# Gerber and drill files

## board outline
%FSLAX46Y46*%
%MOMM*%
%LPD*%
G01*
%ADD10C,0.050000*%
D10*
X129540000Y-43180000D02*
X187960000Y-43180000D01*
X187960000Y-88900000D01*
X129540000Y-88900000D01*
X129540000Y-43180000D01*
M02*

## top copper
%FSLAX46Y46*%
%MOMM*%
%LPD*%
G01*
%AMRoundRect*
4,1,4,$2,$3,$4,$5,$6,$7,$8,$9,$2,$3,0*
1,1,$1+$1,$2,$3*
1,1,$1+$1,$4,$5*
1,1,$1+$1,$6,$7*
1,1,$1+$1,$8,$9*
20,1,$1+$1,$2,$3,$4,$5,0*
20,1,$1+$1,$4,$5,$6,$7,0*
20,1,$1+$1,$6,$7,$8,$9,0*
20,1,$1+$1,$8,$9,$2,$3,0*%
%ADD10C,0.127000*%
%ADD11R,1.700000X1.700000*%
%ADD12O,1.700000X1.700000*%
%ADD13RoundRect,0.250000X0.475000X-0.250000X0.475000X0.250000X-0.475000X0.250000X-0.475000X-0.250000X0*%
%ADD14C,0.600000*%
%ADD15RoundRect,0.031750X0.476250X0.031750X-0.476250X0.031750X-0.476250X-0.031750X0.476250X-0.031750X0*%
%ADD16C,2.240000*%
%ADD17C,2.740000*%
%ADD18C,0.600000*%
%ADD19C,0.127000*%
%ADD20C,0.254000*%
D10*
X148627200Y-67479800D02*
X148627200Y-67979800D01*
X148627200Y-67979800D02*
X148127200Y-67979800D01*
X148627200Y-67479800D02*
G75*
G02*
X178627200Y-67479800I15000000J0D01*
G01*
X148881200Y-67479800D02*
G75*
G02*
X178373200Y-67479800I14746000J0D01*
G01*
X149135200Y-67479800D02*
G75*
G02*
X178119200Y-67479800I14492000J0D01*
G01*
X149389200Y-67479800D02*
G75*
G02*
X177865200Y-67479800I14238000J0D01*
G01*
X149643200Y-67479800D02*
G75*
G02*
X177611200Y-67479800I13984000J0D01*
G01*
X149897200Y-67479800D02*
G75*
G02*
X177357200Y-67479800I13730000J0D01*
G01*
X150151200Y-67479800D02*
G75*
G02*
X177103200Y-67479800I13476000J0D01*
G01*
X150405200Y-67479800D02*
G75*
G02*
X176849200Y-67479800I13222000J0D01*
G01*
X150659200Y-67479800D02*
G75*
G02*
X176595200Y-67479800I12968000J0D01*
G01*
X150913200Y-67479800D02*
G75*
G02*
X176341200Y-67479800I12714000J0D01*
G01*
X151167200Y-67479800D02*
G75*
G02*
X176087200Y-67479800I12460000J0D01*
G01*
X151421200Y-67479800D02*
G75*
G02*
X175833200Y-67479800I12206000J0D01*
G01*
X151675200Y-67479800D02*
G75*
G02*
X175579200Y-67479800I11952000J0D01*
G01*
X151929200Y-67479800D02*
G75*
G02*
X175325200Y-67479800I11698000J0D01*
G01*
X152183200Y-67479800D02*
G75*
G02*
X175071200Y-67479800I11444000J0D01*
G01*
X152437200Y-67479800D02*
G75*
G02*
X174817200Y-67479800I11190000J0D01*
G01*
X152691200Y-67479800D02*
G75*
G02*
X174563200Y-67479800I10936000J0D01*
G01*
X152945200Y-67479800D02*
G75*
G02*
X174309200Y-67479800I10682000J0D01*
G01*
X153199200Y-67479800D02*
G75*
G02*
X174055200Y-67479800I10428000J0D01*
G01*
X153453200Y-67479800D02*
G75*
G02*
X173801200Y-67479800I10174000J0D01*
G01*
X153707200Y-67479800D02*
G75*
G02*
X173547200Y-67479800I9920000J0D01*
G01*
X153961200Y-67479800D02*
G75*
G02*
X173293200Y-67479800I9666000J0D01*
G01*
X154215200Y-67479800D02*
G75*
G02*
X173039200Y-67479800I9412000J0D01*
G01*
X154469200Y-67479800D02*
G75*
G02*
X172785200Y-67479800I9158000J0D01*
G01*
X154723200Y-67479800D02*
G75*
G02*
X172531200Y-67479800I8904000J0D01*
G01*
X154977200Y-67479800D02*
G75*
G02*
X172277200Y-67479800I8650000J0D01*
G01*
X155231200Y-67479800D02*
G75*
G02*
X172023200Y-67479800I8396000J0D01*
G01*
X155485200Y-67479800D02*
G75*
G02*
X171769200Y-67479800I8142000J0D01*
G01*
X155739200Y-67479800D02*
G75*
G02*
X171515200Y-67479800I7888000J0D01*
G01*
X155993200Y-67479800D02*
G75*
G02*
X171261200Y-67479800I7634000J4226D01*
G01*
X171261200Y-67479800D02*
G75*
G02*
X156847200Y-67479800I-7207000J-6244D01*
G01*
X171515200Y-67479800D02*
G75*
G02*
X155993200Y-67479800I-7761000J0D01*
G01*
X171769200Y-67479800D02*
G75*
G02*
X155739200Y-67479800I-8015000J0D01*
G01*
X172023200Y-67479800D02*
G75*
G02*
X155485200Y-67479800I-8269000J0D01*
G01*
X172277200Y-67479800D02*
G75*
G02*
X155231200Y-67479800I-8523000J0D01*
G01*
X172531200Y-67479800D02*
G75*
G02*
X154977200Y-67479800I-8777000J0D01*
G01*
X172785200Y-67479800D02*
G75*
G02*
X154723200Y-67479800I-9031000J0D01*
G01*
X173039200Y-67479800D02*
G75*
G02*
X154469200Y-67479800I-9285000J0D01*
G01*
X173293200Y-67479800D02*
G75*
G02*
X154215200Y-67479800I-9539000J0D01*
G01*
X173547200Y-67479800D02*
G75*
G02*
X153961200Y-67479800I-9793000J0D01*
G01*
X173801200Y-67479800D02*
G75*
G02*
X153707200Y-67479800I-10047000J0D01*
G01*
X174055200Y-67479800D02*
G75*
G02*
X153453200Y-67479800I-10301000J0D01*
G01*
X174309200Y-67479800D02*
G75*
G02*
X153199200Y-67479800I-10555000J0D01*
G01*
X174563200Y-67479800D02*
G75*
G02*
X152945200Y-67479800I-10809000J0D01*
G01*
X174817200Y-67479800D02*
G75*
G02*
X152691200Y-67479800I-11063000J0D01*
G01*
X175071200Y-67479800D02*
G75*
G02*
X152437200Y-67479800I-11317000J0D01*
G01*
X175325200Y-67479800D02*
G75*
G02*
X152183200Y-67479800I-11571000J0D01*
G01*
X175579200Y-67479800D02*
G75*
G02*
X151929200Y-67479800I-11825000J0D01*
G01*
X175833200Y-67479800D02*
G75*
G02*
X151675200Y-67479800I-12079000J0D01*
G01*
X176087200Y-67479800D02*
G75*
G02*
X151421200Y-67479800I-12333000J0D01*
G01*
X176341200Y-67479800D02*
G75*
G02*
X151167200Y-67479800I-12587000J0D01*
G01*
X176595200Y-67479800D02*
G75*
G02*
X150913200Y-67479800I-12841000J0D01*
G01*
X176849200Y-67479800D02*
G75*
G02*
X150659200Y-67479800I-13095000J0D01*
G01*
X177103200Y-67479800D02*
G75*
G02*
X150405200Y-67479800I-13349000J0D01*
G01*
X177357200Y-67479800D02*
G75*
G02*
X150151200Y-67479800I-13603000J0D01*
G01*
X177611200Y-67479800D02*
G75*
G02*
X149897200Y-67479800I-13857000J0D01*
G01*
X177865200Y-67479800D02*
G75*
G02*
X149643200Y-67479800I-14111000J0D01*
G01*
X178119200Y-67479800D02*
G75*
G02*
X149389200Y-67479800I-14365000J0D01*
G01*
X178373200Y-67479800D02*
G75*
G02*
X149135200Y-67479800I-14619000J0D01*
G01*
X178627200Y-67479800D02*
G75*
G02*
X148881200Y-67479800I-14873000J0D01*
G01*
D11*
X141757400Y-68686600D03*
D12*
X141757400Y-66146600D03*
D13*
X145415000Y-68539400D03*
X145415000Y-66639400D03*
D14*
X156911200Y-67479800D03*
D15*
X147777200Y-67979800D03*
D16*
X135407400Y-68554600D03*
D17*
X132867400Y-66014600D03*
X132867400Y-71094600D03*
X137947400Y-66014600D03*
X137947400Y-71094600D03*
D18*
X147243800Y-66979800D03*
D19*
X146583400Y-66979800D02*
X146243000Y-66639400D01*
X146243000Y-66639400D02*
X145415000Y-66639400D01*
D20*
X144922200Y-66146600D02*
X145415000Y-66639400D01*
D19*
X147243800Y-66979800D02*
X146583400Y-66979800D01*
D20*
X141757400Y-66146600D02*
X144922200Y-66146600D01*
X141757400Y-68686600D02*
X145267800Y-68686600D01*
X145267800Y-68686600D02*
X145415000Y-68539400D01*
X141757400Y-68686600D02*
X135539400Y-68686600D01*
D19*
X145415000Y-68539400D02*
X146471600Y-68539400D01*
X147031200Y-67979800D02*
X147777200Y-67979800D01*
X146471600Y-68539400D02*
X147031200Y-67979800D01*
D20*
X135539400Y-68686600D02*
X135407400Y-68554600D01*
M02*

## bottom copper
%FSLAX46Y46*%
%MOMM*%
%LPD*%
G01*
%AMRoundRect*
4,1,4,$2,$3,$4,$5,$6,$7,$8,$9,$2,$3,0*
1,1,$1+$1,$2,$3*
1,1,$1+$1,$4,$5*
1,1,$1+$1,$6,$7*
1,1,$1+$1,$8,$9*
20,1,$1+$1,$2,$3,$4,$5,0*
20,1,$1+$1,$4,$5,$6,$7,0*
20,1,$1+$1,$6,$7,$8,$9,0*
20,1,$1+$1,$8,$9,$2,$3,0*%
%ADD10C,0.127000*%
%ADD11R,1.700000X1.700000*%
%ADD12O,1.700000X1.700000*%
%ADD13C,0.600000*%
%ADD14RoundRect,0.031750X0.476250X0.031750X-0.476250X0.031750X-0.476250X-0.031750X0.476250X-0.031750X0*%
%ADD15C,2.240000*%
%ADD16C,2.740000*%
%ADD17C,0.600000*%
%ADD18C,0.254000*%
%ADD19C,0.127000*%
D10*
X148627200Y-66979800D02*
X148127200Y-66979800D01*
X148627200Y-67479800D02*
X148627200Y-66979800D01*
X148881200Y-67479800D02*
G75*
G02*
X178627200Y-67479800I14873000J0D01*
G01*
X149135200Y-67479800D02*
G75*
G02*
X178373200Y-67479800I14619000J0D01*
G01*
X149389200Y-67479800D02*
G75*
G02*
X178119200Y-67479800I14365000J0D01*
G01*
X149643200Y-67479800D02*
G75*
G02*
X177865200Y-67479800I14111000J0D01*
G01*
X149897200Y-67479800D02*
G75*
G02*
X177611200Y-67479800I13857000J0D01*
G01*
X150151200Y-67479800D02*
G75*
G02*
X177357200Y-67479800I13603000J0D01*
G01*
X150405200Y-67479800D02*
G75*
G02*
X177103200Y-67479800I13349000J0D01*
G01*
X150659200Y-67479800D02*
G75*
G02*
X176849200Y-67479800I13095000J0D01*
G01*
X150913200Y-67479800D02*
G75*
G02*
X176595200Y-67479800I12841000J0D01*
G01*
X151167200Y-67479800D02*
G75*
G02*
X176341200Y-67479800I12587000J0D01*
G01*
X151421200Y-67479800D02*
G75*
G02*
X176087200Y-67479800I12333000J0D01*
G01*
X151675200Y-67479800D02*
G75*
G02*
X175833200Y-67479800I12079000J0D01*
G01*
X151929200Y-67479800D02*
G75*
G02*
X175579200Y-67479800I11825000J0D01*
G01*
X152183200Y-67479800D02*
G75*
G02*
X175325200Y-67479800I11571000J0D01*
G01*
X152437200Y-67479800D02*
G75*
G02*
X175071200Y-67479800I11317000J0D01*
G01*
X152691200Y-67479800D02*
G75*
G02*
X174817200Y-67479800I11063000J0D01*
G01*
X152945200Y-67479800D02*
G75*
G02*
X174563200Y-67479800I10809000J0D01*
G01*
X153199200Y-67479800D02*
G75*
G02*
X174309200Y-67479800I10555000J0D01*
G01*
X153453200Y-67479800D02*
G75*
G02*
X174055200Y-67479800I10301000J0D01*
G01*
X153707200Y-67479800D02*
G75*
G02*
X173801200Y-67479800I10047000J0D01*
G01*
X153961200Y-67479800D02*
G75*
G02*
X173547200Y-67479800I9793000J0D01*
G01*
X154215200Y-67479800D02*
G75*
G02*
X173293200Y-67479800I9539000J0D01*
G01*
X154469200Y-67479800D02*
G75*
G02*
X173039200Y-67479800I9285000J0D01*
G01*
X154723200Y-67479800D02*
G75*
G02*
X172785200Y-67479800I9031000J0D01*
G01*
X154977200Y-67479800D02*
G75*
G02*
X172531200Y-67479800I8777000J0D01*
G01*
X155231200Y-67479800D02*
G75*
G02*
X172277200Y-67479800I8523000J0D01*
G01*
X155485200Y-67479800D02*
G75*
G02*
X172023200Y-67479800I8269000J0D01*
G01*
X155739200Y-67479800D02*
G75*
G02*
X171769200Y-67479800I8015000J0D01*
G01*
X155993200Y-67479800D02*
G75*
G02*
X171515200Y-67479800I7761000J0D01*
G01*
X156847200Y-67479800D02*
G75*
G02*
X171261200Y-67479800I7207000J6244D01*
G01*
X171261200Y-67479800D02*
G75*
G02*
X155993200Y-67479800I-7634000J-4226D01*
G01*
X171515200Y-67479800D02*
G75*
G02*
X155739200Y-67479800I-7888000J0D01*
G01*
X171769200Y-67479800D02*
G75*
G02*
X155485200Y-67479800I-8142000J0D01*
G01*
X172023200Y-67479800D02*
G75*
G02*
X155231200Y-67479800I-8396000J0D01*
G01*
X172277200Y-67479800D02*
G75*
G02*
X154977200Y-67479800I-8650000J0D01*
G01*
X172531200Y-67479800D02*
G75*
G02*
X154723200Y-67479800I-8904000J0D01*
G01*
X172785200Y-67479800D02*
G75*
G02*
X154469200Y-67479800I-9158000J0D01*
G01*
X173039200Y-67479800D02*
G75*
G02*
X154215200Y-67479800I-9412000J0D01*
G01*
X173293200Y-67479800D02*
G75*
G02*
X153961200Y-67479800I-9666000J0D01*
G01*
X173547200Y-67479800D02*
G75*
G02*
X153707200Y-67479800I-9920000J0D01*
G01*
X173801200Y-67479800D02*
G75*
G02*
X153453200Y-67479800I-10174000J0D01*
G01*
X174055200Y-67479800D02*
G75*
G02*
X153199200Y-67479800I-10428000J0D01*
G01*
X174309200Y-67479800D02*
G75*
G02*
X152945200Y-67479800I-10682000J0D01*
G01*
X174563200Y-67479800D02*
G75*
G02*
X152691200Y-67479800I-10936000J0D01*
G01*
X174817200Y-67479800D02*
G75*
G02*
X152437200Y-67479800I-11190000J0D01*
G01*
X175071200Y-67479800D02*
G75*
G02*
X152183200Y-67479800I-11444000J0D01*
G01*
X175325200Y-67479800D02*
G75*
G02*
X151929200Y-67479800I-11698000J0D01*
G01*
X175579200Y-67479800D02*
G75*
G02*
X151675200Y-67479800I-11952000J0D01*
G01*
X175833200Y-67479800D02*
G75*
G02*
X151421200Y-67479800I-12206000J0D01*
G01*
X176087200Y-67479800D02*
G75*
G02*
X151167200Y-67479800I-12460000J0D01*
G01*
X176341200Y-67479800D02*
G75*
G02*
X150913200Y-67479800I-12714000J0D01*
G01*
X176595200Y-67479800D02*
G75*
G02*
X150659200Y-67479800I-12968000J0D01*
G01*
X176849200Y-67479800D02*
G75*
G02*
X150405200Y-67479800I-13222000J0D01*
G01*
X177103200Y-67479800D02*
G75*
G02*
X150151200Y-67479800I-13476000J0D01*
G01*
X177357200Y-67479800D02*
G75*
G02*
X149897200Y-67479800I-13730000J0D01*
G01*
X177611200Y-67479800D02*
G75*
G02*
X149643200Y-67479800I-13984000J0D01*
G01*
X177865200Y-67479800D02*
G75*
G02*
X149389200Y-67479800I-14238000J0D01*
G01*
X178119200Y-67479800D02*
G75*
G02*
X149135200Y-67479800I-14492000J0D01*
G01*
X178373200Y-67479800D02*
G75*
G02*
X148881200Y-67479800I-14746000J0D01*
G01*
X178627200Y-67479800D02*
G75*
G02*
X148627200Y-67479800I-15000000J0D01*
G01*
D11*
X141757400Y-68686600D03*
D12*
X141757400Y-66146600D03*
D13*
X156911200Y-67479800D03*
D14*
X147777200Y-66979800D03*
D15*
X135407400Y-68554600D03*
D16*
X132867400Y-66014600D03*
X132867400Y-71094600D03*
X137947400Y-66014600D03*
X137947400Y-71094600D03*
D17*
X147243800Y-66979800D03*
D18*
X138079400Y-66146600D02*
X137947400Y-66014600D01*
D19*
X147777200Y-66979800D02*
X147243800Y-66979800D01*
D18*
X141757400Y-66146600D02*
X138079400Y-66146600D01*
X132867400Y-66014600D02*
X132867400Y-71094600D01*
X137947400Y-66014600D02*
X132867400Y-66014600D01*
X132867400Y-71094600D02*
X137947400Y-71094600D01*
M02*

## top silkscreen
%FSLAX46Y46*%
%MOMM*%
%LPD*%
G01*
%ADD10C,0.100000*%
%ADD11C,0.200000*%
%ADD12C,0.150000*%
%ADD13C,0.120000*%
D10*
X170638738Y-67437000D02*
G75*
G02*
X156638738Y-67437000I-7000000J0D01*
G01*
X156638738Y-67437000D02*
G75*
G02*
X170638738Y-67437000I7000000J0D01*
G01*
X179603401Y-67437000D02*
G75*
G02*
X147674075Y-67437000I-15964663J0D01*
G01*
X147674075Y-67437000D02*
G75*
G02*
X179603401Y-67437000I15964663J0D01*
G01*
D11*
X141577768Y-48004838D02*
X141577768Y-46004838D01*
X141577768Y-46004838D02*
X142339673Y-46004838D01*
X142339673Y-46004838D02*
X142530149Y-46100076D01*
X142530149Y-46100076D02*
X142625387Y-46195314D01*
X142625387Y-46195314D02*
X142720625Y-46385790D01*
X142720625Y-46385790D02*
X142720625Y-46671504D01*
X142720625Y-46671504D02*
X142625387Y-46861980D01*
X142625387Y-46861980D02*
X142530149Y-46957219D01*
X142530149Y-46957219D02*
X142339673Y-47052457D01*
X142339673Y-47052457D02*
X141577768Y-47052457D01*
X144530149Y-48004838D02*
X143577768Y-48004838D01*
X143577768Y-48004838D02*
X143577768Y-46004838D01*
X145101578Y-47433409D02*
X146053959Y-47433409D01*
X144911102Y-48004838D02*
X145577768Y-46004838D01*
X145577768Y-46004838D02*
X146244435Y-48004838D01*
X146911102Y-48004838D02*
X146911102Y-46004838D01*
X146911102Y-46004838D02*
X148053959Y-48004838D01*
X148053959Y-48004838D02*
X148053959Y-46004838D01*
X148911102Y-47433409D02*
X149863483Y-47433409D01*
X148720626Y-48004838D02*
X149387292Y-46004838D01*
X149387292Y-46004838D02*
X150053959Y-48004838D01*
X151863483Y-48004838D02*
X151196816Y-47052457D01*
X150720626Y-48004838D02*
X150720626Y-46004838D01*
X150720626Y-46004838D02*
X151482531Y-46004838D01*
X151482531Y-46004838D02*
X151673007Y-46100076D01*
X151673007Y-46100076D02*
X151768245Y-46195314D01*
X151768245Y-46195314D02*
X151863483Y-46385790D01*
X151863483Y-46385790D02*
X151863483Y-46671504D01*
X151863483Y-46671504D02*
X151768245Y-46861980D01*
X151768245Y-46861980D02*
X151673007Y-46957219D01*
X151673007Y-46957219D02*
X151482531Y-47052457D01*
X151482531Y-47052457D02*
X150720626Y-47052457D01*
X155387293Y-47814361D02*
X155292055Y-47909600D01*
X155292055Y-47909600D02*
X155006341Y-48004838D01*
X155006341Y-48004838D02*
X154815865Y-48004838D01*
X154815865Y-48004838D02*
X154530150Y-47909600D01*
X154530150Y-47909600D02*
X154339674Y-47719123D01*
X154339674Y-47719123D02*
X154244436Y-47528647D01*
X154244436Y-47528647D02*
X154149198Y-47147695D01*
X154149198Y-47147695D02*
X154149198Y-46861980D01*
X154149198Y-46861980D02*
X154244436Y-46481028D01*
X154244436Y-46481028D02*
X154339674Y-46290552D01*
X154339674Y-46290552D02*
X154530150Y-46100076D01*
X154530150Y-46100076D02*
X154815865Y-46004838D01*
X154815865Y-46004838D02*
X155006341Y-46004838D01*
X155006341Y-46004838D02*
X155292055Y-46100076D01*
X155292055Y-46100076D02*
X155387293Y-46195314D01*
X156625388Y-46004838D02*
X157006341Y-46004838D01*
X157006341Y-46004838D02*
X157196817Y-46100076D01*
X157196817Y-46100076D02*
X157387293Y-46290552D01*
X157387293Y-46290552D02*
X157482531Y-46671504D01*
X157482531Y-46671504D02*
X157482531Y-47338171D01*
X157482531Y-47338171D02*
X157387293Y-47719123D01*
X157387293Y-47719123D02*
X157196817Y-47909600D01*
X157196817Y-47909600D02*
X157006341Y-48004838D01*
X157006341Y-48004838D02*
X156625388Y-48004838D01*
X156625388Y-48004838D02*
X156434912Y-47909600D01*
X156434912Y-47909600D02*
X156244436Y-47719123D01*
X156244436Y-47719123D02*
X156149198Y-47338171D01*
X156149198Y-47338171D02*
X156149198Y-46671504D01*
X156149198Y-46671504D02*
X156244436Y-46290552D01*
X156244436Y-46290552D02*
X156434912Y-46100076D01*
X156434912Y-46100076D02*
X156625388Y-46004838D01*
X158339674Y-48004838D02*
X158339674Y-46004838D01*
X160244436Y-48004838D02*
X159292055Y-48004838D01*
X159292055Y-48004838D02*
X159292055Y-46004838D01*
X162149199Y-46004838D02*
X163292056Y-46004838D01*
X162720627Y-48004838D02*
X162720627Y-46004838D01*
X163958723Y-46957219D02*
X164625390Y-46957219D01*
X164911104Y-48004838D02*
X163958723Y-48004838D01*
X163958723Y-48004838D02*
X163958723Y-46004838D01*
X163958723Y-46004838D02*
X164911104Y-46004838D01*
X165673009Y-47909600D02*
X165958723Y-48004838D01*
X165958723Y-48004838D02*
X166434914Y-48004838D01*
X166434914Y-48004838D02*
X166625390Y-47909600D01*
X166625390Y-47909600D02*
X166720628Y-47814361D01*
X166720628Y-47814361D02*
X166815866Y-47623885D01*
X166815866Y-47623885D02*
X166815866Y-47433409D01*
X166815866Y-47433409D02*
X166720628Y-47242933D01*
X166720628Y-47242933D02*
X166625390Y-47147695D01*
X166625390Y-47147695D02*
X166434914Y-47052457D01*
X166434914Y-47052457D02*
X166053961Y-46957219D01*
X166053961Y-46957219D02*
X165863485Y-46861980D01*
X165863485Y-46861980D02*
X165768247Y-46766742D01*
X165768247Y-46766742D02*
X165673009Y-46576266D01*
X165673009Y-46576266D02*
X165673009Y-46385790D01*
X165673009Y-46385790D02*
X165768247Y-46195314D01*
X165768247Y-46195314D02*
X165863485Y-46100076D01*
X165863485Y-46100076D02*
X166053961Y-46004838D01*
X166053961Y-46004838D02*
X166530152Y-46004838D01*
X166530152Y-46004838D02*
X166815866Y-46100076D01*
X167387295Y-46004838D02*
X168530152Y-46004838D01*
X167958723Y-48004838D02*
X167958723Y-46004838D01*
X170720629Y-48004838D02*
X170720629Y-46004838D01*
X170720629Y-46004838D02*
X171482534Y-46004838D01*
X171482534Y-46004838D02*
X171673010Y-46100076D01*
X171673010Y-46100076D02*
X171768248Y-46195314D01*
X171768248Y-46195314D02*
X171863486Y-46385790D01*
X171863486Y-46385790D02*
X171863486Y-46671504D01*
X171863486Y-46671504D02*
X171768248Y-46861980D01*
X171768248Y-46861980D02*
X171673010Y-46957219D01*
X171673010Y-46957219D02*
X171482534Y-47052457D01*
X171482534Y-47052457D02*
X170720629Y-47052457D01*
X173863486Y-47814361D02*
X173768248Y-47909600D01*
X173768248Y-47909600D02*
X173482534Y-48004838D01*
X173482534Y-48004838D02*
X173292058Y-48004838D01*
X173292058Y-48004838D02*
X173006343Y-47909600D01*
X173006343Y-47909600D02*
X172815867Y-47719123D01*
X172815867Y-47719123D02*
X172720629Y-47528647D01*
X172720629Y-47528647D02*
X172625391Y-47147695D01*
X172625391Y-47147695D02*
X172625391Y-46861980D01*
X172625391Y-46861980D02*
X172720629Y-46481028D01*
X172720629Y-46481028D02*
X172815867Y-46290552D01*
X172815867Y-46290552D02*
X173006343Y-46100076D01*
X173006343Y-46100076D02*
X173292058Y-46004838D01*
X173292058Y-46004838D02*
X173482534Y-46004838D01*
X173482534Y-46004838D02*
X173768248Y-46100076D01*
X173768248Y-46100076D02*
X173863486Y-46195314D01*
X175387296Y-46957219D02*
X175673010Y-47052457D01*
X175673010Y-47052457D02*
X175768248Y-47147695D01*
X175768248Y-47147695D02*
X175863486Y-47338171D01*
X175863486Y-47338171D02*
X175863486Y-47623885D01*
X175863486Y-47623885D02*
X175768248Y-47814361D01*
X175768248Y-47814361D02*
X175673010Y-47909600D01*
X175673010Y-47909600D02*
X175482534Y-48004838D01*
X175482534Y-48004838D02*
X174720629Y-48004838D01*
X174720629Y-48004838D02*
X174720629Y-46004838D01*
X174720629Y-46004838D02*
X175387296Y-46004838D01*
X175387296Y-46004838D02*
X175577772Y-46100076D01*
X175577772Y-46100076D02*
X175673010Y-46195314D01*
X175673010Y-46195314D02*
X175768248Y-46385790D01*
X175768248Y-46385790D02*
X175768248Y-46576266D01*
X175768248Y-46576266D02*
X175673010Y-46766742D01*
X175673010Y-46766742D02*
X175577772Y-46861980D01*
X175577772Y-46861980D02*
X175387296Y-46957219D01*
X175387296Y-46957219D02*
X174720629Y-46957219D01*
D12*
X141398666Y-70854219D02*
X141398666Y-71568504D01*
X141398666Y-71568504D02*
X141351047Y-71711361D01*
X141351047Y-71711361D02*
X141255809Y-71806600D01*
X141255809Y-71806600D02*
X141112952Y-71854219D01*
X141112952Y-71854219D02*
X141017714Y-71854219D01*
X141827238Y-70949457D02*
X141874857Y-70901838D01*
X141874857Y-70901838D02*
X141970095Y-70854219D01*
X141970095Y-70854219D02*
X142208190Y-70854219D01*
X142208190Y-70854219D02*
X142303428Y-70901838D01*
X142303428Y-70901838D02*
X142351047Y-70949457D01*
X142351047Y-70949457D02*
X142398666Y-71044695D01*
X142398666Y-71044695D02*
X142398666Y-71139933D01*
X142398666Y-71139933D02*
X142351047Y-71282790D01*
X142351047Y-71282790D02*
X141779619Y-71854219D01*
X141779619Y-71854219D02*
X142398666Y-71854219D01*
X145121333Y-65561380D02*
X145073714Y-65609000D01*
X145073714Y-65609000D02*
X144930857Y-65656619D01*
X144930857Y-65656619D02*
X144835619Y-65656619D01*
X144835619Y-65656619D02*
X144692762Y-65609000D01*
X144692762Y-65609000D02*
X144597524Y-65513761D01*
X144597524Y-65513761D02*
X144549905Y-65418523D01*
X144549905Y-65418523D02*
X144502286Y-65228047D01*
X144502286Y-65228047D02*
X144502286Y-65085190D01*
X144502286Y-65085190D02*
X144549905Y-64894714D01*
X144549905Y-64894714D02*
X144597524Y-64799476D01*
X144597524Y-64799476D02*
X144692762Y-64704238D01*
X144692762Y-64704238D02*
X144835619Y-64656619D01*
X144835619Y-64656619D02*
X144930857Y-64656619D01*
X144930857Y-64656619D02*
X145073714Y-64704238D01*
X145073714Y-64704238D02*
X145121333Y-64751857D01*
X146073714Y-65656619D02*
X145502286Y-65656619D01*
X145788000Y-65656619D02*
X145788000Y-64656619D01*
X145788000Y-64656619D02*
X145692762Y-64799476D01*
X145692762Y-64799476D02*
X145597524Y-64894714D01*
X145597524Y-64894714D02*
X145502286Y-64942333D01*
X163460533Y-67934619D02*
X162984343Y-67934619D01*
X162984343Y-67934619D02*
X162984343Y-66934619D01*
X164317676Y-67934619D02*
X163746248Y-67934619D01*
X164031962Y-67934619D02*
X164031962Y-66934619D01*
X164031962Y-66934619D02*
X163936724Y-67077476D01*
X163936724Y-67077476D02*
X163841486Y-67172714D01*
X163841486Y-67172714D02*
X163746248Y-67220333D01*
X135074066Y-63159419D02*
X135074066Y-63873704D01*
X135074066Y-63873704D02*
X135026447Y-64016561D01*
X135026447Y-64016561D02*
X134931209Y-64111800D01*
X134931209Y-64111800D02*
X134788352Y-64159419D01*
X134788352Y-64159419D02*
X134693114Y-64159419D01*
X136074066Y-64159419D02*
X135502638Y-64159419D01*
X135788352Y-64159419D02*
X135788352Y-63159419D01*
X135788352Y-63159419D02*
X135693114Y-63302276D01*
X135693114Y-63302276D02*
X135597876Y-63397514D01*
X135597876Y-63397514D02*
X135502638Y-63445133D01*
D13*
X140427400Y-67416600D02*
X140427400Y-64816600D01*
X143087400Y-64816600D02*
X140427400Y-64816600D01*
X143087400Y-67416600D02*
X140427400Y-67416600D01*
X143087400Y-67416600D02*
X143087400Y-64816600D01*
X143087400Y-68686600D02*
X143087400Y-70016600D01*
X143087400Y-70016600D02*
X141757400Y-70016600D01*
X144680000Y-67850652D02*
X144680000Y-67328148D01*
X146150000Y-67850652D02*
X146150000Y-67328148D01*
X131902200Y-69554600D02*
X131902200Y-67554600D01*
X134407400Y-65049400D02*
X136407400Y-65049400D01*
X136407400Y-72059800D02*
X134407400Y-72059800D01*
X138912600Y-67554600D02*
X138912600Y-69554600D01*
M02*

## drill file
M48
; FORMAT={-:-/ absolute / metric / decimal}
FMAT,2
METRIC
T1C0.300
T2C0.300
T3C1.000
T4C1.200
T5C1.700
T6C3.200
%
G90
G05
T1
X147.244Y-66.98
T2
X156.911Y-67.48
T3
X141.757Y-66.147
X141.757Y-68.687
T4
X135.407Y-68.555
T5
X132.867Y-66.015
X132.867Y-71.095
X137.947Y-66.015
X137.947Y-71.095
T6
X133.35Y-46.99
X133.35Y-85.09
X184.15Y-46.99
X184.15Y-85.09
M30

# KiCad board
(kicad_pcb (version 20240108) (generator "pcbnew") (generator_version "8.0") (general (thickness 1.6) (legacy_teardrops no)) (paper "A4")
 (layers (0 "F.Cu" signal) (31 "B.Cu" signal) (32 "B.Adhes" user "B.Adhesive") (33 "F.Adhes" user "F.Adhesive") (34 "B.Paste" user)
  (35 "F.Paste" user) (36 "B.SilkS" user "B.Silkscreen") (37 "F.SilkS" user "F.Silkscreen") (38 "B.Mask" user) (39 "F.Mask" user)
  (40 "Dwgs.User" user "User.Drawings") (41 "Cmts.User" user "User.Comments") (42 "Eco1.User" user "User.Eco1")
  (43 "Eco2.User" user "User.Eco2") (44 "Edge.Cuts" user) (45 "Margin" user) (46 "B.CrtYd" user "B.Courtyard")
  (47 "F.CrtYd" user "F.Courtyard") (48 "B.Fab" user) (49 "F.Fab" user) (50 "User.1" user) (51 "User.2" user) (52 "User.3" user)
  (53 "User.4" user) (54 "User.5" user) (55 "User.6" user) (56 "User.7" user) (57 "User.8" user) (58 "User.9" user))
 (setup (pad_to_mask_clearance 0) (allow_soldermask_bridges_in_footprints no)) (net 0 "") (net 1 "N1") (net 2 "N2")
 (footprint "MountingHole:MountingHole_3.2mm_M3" (layer "F.Cu") (at 184.15 85.09)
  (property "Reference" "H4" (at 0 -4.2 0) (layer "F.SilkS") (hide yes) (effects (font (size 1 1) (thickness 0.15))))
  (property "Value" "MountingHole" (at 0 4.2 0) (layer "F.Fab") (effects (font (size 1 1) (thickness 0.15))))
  (pad "" np_thru_hole circle (at 0 0) (size 3.2 3.2) (drill 3.2) (layers "*.Cu" "*.Mask")))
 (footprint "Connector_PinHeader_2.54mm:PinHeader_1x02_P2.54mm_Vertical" (layer "F.Cu") (at 141.7574 68.6866 180)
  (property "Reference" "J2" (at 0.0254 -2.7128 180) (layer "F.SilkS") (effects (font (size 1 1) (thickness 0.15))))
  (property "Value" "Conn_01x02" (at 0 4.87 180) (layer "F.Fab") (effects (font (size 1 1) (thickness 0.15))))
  (fp_line (start 1.33 1.27) (end 1.33 3.87) (stroke (width 0.12) (type solid)) (layer "F.SilkS"))
  (fp_line (start -1.33 3.87) (end 1.33 3.87) (stroke (width 0.12) (type solid)) (layer "F.SilkS"))
  (fp_line (start -1.33 1.27) (end 1.33 1.27) (stroke (width 0.12) (type solid)) (layer "F.SilkS"))
  (fp_line (start -1.33 1.27) (end -1.33 3.87) (stroke (width 0.12) (type solid)) (layer "F.SilkS"))
  (fp_line (start -1.33 0) (end -1.33 -1.33) (stroke (width 0.12) (type solid)) (layer "F.SilkS"))
  (fp_line (start -1.33 -1.33) (end 0 -1.33) (stroke (width 0.12) (type solid)) (layer "F.SilkS"))
  (pad "1" thru_hole rect (at 0 0 180) (size 1.7 1.7) (drill 1) (layers "*.Cu" "*.Mask") (remove_unused_layers no) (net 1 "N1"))
  (pad "2" thru_hole oval (at 0 2.54 180) (size 1.7 1.7) (drill 1) (layers "*.Cu" "*.Mask") (remove_unused_layers no) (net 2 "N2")))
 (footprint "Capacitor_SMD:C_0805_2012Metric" (layer "F.Cu") (at 145.415 67.5894 90)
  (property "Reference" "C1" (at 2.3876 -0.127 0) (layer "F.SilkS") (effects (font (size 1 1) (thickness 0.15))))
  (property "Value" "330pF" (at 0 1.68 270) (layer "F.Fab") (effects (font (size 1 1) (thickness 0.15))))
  (fp_line (start -0.261252 -0.735) (end 0.261252 -0.735) (stroke (width 0.12) (type solid)) (layer "F.SilkS"))
  (fp_line (start -0.261252 0.735) (end 0.261252 0.735) (stroke (width 0.12) (type solid)) (layer "F.SilkS"))
  (pad "1" smd roundrect (at -0.95 0 90) (size 1 1.45) (layers "F.Cu" "F.Paste" "F.Mask") (roundrect_rratio 0.25) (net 1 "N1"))
  (pad "2" smd roundrect (at 0.95 0 90) (size 1 1.45) (layers "F.Cu" "F.Paste" "F.Mask") (roundrect_rratio 0.25) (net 2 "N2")))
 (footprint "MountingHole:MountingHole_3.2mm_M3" (layer "F.Cu") (at 133.35 46.99)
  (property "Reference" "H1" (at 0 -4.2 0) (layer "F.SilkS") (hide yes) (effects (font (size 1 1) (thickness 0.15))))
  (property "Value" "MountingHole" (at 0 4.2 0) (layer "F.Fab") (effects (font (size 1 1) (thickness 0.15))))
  (pad "" np_thru_hole circle (at 0 0) (size 3.2 3.2) (drill 3.2) (layers "*.Cu" "*.Mask")))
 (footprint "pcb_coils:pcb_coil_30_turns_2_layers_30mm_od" (layer "F.Cu") (at 163.7542 67.4798 180)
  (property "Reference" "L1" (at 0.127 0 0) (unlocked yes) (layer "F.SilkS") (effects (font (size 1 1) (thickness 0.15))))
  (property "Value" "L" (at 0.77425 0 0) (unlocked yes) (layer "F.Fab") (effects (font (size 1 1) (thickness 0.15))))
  (fp_line (start 15.127 0) (end 15.127 -0.5) (stroke (width 0.127) (type solid)) (layer "F.Cu"))
  (fp_line (start 15.127 -0.5) (end 15.627 -0.5) (stroke (width 0.127) (type solid)) (layer "F.Cu"))
  (fp_arc (start 15.127 0) (mid 0.127 15) (end -14.873 0) (stroke (width 0.127) (type solid)) (layer "F.Cu"))
  (fp_arc (start 14.873 0) (mid 0.127 14.746) (end -14.619 0) (stroke (width 0.127) (type solid)) (layer "F.Cu"))
  (fp_arc (start 14.619 0) (mid 0.127 14.492) (end -14.365 0) (stroke (width 0.127) (type solid)) (layer "F.Cu"))
  (fp_arc (start 14.365 0) (mid 0.127 14.238) (end -14.111 0) (stroke (width 0.127) (type solid)) (layer "F.Cu"))
  (fp_arc (start 14.111 0) (mid 0.127 13.984) (end -13.857 0) (stroke (width 0.127) (type solid)) (layer "F.Cu"))
  (fp_arc (start 13.857 0) (mid 0.127 13.73) (end -13.603 0) (stroke (width 0.127) (type solid)) (layer "F.Cu"))
  (fp_arc (start 13.603 0) (mid 0.127 13.476) (end -13.349 0) (stroke (width 0.127) (type solid)) (layer "F.Cu"))
  (fp_arc (start 13.349 0) (mid 0.127 13.222) (end -13.095 0) (stroke (width 0.127) (type solid)) (layer "F.Cu"))
  (fp_arc (start 13.095 0) (mid 0.127 12.968) (end -12.841 0) (stroke (width 0.127) (type solid)) (layer "F.Cu"))
  (fp_arc (start 12.841 0) (mid 0.127 12.714) (end -12.587 0) (stroke (width 0.127) (type solid)) (layer "F.Cu"))
  (fp_arc (start 12.587 0) (mid 0.127 12.46) (end -12.333 0) (stroke (width 0.127) (type solid)) (layer "F.Cu"))
  (fp_arc (start 12.333 0) (mid 0.127 12.206) (end -12.079 0) (stroke (width 0.127) (type solid)) (layer "F.Cu"))
  (fp_arc (start 12.079 0) (mid 0.127 11.952) (end -11.825 0) (stroke (width 0.127) (type solid)) (layer "F.Cu"))
  (fp_arc (start 11.825 0) (mid 0.127 11.698) (end -11.571 0) (stroke (width 0.127) (type solid)) (layer "F.Cu"))
  (fp_arc (start 11.571 0) (mid 0.127 11.444) (end -11.317 0) (stroke (width 0.127) (type solid)) (layer "F.Cu"))
  (fp_arc (start 11.317 0) (mid 0.127 11.19) (end -11.063 0) (stroke (width 0.127) (type solid)) (layer "F.Cu"))
  (fp_arc (start 11.063 0) (mid 0.127 10.936) (end -10.809 0) (stroke (width 0.127) (type solid)) (layer "F.Cu"))
  (fp_arc (start 10.809 0) (mid 0.127 10.682) (end -10.555 0) (stroke (width 0.127) (type solid)) (layer "F.Cu"))
  (fp_arc (start 10.555 0) (mid 0.127 10.428) (end -10.301 0) (stroke (width 0.127) (type solid)) (layer "F.Cu"))
  (fp_arc (start 10.301 0) (mid 0.127 10.174) (end -10.047 0) (stroke (width 0.127) (type solid)) (layer "F.Cu"))
  (fp_arc (start 10.047 0) (mid 0.127 9.92) (end -9.793 0) (stroke (width 0.127) (type solid)) (layer "F.Cu"))
  (fp_arc (start 9.793 0) (mid 0.127 9.666) (end -9.539 0) (stroke (width 0.127) (type solid)) (layer "F.Cu"))
  (fp_arc (start 9.539 0) (mid 0.127 9.412) (end -9.285 0) (stroke (width 0.127) (type solid)) (layer "F.Cu"))
  (fp_arc (start 9.285 0) (mid 0.127 9.158) (end -9.031 0) (stroke (width 0.127) (type solid)) (layer "F.Cu"))
  (fp_arc (start 9.031 0) (mid 0.127 8.904) (end -8.777 0) (stroke (width 0.127) (type solid)) (layer "F.Cu"))
  (fp_arc (start 8.777 0) (mid 0.127 8.65) (end -8.523 0) (stroke (width 0.127) (type solid)) (layer "F.Cu"))
  (fp_arc (start 8.523 0) (mid 0.127 8.396) (end -8.269 0) (stroke (width 0.127) (type solid)) (layer "F.Cu"))
  (fp_arc (start 8.269 0) (mid 0.127 8.142) (end -8.015 0) (stroke (width 0.127) (type solid)) (layer "F.Cu"))
  (fp_arc (start 8.015 0) (mid 0.127 7.888) (end -7.761 0) (stroke (width 0.127) (type solid)) (layer "F.Cu"))
  (fp_arc (start 7.761 0) (mid 0.127 7.638227) (end -7.507 0) (stroke (width 0.127) (type solid)) (layer "F.Cu"))
  (fp_arc (start -7.507 0) (mid -0.3 -7.213247) (end 6.907 0) (stroke (width 0.127) (type solid)) (layer "F.Cu"))
  (fp_arc (start -7.761 0) (mid 0 -7.761) (end 7.761 0) (stroke (width 0.127) (type solid)) (layer "F.Cu"))
  (fp_arc (start -8.015 0) (mid 0 -8.015) (end 8.015 0) (stroke (width 0.127) (type solid)) (layer "F.Cu"))
  (fp_arc (start -8.269 0) (mid 0 -8.269) (end 8.269 0) (stroke (width 0.127) (type solid)) (layer "F.Cu"))
  (fp_arc (start -8.523 0) (mid 0 -8.523) (end 8.523 0) (stroke (width 0.127) (type solid)) (layer "F.Cu"))
  (fp_arc (start -8.777 0) (mid 0 -8.777) (end 8.777 0) (stroke (width 0.127) (type solid)) (layer "F.Cu"))
  (fp_arc (start -9.031 0) (mid 0 -9.031) (end 9.031 0) (stroke (width 0.127) (type solid)) (layer "F.Cu"))
  (fp_arc (start -9.285 0) (mid 0 -9.285) (end 9.285 0) (stroke (width 0.127) (type solid)) (layer "F.Cu"))
  (fp_arc (start -9.539 0) (mid 0 -9.539) (end 9.539 0) (stroke (width 0.127) (type solid)) (layer "F.Cu"))
  (fp_arc (start -9.793 0) (mid 0 -9.793) (end 9.793 0) (stroke (width 0.127) (type solid)) (layer "F.Cu"))
  (fp_arc (start -10.047 0) (mid 0 -10.047) (end 10.047 0) (stroke (width 0.127) (type solid)) (layer "F.Cu"))
  (fp_arc (start -10.301 0) (mid 0 -10.301) (end 10.301 0) (stroke (width 0.127) (type solid)) (layer "F.Cu"))
  (fp_arc (start -10.555 0) (mid 0 -10.555) (end 10.555 0) (stroke (width 0.127) (type solid)) (layer "F.Cu"))
  (fp_arc (start -10.809 0) (mid 0 -10.809) (end 10.809 0) (stroke (width 0.127) (type solid)) (layer "F.Cu"))
  (fp_arc (start -11.063 0) (mid 0 -11.063) (end 11.063 0) (stroke (width 0.127) (type solid)) (layer "F.Cu"))
  (fp_arc (start -11.317 0) (mid 0 -11.317) (end 11.317 0) (stroke (width 0.127) (type solid)) (layer "F.Cu"))
  (fp_arc (start -11.571 0) (mid 0 -11.571) (end 11.571 0) (stroke (width 0.127) (type solid)) (layer "F.Cu"))
  (fp_arc (start -11.825 0) (mid 0 -11.825) (end 11.825 0) (stroke (width 0.127) (type solid)) (layer "F.Cu"))
  (fp_arc (start -12.079 0) (mid 0 -12.079) (end 12.079 0) (stroke (width 0.127) (type solid)) (layer "F.Cu"))
  (fp_arc (start -12.333 0) (mid 0 -12.333) (end 12.333 0) (stroke (width 0.127) (type solid)) (layer "F.Cu"))
  (fp_arc (start -12.587 0) (mid 0 -12.587) (end 12.587 0) (stroke (width 0.127) (type solid)) (layer "F.Cu"))
  (fp_arc (start -12.841 0) (mid 0 -12.841) (end 12.841 0) (stroke (width 0.127) (type solid)) (layer "F.Cu"))
  (fp_arc (start -13.095 0) (mid 0 -13.095) (end 13.095 0) (stroke (width 0.127) (type solid)) (layer "F.Cu"))
  (fp_arc (start -13.349 0) (mid 0 -13.349) (end 13.349 0) (stroke (width 0.127) (type solid)) (layer "F.Cu"))
  (fp_arc (start -13.603 0) (mid 0 -13.603) (end 13.603 0) (stroke (width 0.127) (type solid)) (layer "F.Cu"))
  (fp_arc (start -13.857 0) (mid 0 -13.857) (end 13.857 0) (stroke (width 0.127) (type solid)) (layer "F.Cu"))
  (fp_arc (start -14.111 0) (mid 0 -14.111) (end 14.111 0) (stroke (width 0.127) (type solid)) (layer "F.Cu"))
  (fp_arc (start -14.365 0) (mid 0 -14.365) (end 14.365 0) (stroke (width 0.127) (type solid)) (layer "F.Cu"))
  (fp_arc (start -14.619 0) (mid 0 -14.619) (end 14.619 0) (stroke (width 0.127) (type solid)) (layer "F.Cu"))
  (fp_arc (start -14.873 0) (mid 0 -14.873) (end 14.873 0) (stroke (width 0.127) (type solid)) (layer "F.Cu"))
  (fp_line (start 15.127 0.5) (end 15.627 0.5) (stroke (width 0.127) (type solid)) (layer "B.Cu"))
  (fp_line (start 15.127 0) (end 15.127 0.5) (stroke (width 0.127) (type solid)) (layer "B.Cu"))
  (fp_arc (start 14.873 0) (mid 0 14.873) (end -14.873 0) (stroke (width 0.127) (type solid)) (layer "B.Cu"))
  (fp_arc (start 14.619 0) (mid 0 14.619) (end -14.619 0) (stroke (width 0.127) (type solid)) (layer "B.Cu"))
  (fp_arc (start 14.365 0) (mid 0 14.365) (end -14.365 0) (stroke (width 0.127) (type solid)) (layer "B.Cu"))
  (fp_arc (start 14.111 0) (mid 0 14.111) (end -14.111 0) (stroke (width 0.127) (type solid)) (layer "B.Cu"))
  (fp_arc (start 13.857 0) (mid 0 13.857) (end -13.857 0) (stroke (width 0.127) (type solid)) (layer "B.Cu"))
  (fp_arc (start 13.603 0) (mid 0 13.603) (end -13.603 0) (stroke (width 0.127) (type solid)) (layer "B.Cu"))
  (fp_arc (start 13.349 0) (mid 0 13.349) (end -13.349 0) (stroke (width 0.127) (type solid)) (layer "B.Cu"))
  (fp_arc (start 13.095 0) (mid 0 13.095) (end -13.095 0) (stroke (width 0.127) (type solid)) (layer "B.Cu"))
  (fp_arc (start 12.841 0) (mid 0 12.841) (end -12.841 0) (stroke (width 0.127) (type solid)) (layer "B.Cu"))
  (fp_arc (start 12.587 0) (mid 0 12.587) (end -12.587 0) (stroke (width 0.127) (type solid)) (layer "B.Cu"))
  (fp_arc (start 12.333 0) (mid 0 12.333) (end -12.333 0) (stroke (width 0.127) (type solid)) (layer "B.Cu"))
  (fp_arc (start 12.079 0) (mid 0 12.079) (end -12.079 0) (stroke (width 0.127) (type solid)) (layer "B.Cu"))
  (fp_arc (start 11.825 0) (mid 0 11.825) (end -11.825 0) (stroke (width 0.127) (type solid)) (layer "B.Cu"))
  (fp_arc (start 11.571 0) (mid 0 11.571) (end -11.571 0) (stroke (width 0.127) (type solid)) (layer "B.Cu"))
  (fp_arc (start 11.317 0) (mid 0 11.317) (end -11.317 0) (stroke (width 0.127) (type solid)) (layer "B.Cu"))
  (fp_arc (start 11.063 0) (mid 0 11.063) (end -11.063 0) (stroke (width 0.127) (type solid)) (layer "B.Cu"))
  (fp_arc (start 10.809 0) (mid 0 10.809) (end -10.809 0) (stroke (width 0.127) (type solid)) (layer "B.Cu"))
  (fp_arc (start 10.555 0) (mid 0 10.555) (end -10.555 0) (stroke (width 0.127) (type solid)) (layer "B.Cu"))
  (fp_arc (start 10.301 0) (mid 0 10.301) (end -10.301 0) (stroke (width 0.127) (type solid)) (layer "B.Cu"))
  (fp_arc (start 10.047 0) (mid 0 10.047) (end -10.047 0) (stroke (width 0.127) (type solid)) (layer "B.Cu"))
  (fp_arc (start 9.793 0) (mid 0 9.793) (end -9.793 0) (stroke (width 0.127) (type solid)) (layer "B.Cu"))
  (fp_arc (start 9.539 0) (mid 0 9.539) (end -9.539 0) (stroke (width 0.127) (type solid)) (layer "B.Cu"))
  (fp_arc (start 9.285 0) (mid 0 9.285) (end -9.285 0) (stroke (width 0.127) (type solid)) (layer "B.Cu"))
  (fp_arc (start 9.031 0) (mid 0 9.031) (end -9.031 0) (stroke (width 0.127) (type solid)) (layer "B.Cu"))
  (fp_arc (start 8.777 0) (mid 0 8.777) (end -8.777 0) (stroke (width 0.127) (type solid)) (layer "B.Cu"))
  (fp_arc (start 8.523 0) (mid 0 8.523) (end -8.523 0) (stroke (width 0.127) (type solid)) (layer "B.Cu"))
  (fp_arc (start 8.269 0) (mid 0 8.269) (end -8.269 0) (stroke (width 0.127) (type solid)) (layer "B.Cu"))
  (fp_arc (start 8.015 0) (mid 0 8.015) (end -8.015 0) (stroke (width 0.127) (type solid)) (layer "B.Cu"))
  (fp_arc (start 7.761 0) (mid 0 7.761) (end -7.761 0) (stroke (width 0.127) (type solid)) (layer "B.Cu"))
  (fp_arc (start 6.907 0) (mid -0.3 7.213247) (end -7.507 0) (stroke (width 0.127) (type solid)) (layer "B.Cu"))
  (fp_arc (start -7.507 0) (mid 0.127 -7.638227) (end 7.761 0) (stroke (width 0.127) (type solid)) (layer "B.Cu"))
  (fp_arc (start -7.761 0) (mid 0.127 -7.888) (end 8.015 0) (stroke (width 0.127) (type solid)) (layer "B.Cu"))
  (fp_arc (start -8.015 0) (mid 0.127 -8.142) (end 8.269 0) (stroke (width 0.127) (type solid)) (layer "B.Cu"))
  (fp_arc (start -8.269 0) (mid 0.127 -8.396) (end 8.523 0) (stroke (width 0.127) (type solid)) (layer "B.Cu"))
  (fp_arc (start -8.523 0) (mid 0.127 -8.65) (end 8.777 0) (stroke (width 0.127) (type solid)) (layer "B.Cu"))
  (fp_arc (start -8.777 0) (mid 0.127 -8.904) (end 9.031 0) (stroke (width 0.127) (type solid)) (layer "B.Cu"))
  (fp_arc (start -9.031 0) (mid 0.127 -9.158) (end 9.285 0) (stroke (width 0.127) (type solid)) (layer "B.Cu"))
  (fp_arc (start -9.285 0) (mid 0.127 -9.412) (end 9.539 0) (stroke (width 0.127) (type solid)) (layer "B.Cu"))
  (fp_arc (start -9.539 0) (mid 0.127 -9.666) (end 9.793 0) (stroke (width 0.127) (type solid)) (layer "B.Cu"))
  (fp_arc (start -9.793 0) (mid 0.127 -9.92) (end 10.047 0) (stroke (width 0.127) (type solid)) (layer "B.Cu"))
  (fp_arc (start -10.047 0) (mid 0.127 -10.174) (end 10.301 0) (stroke (width 0.127) (type solid)) (layer "B.Cu"))
  (fp_arc (start -10.301 0) (mid 0.127 -10.428) (end 10.555 0) (stroke (width 0.127) (type solid)) (layer "B.Cu"))
  (fp_arc (start -10.555 0) (mid 0.127 -10.682) (end 10.809 0) (stroke (width 0.127) (type solid)) (layer "B.Cu"))
  (fp_arc (start -10.809 0) (mid 0.127 -10.936) (end 11.063 0) (stroke (width 0.127) (type solid)) (layer "B.Cu"))
  (fp_arc (start -11.063 0) (mid 0.127 -11.19) (end 11.317 0) (stroke (width 0.127) (type solid)) (layer "B.Cu"))
  (fp_arc (start -11.317 0) (mid 0.127 -11.444) (end 11.571 0) (stroke (width 0.127) (type solid)) (layer "B.Cu"))
  (fp_arc (start -11.571 0) (mid 0.127 -11.698) (end 11.825 0) (stroke (width 0.127) (type solid)) (layer "B.Cu"))
  (fp_arc (start -11.825 0) (mid 0.127 -11.952) (end 12.079 0) (stroke (width 0.127) (type solid)) (layer "B.Cu"))
  (fp_arc (start -12.079 0) (mid 0.127 -12.206) (end 12.333 0) (stroke (width 0.127) (type solid)) (layer "B.Cu"))
  (fp_arc (start -12.333 0) (mid 0.127 -12.46) (end 12.587 0) (stroke (width 0.127) (type solid)) (layer "B.Cu"))
  (fp_arc (start -12.587 0) (mid 0.127 -12.714) (end 12.841 0) (stroke (width 0.127) (type solid)) (layer "B.Cu"))
  (fp_arc (start -12.841 0) (mid 0.127 -12.968) (end 13.095 0) (stroke (width 0.127) (type solid)) (layer "B.Cu"))
  (fp_arc (start -13.095 0) (mid 0.127 -13.222) (end 13.349 0) (stroke (width 0.127) (type solid)) (layer "B.Cu"))
  (fp_arc (start -13.349 0) (mid 0.127 -13.476) (end 13.603 0) (stroke (width 0.127) (type solid)) (layer "B.Cu"))
  (fp_arc (start -13.603 0) (mid 0.127 -13.73) (end 13.857 0) (stroke (width 0.127) (type solid)) (layer "B.Cu"))
  (fp_arc (start -13.857 0) (mid 0.127 -13.984) (end 14.111 0) (stroke (width 0.127) (type solid)) (layer "B.Cu"))
  (fp_arc (start -14.111 0) (mid 0.127 -14.238) (end 14.365 0) (stroke (width 0.127) (type solid)) (layer "B.Cu"))
  (fp_arc (start -14.365 0) (mid 0.127 -14.492) (end 14.619 0) (stroke (width 0.127) (type solid)) (layer "B.Cu"))
  (fp_arc (start -14.619 0) (mid 0.127 -14.746) (end 14.873 0) (stroke (width 0.127) (type solid)) (layer "B.Cu"))
  (fp_arc (start -14.873 0) (mid 0.127 -15) (end 15.127 0) (stroke (width 0.127) (type solid)) (layer "B.Cu"))
  (pad "" thru_hole circle (at 6.843 0 180) (size 0.6 0.6) (drill 0.3) (layers "*.Cu" "*.Mask") (remove_unused_layers no))
  (pad "1" smd roundrect (at 15.977 -0.5 180) (size 1.016 0.127) (layers "F.Cu") (roundrect_rratio 0.25) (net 1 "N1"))
  (pad "2" smd roundrect (at 15.977 0.5 180) (size 1.016 0.127) (layers "B.Cu") (roundrect_rratio 0.25) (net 2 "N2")))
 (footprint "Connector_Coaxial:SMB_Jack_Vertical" (layer "F.Cu") (at 135.4074 68.5546)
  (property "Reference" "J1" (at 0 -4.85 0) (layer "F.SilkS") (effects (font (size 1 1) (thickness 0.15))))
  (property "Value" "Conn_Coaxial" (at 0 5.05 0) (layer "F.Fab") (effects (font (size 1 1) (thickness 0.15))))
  (fp_line (start -3.5052 1) (end -3.5052 -1) (stroke (width 0.12) (type solid)) (layer "F.SilkS"))
  (fp_line (start -1 -3.5052) (end 1 -3.5052) (stroke (width 0.12) (type solid)) (layer "F.SilkS"))
  (fp_line (start 1 3.5052) (end -1 3.5052) (stroke (width 0.12) (type solid)) (layer "F.SilkS"))
  (fp_line (start 3.5052 -1) (end 3.5052 1) (stroke (width 0.12) (type solid)) (layer "F.SilkS"))
  (pad "1" thru_hole circle (at 0 0) (size 2.24 2.24) (drill 1.2) (layers "*.Cu" "*.Mask") (remove_unused_layers no) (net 1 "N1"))
  (pad "2" thru_hole circle (at -2.54 -2.54) (size 2.74 2.74) (drill 1.7) (layers "*.Cu" "*.Mask") (remove_unused_layers no) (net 2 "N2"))
  (pad "2" thru_hole circle (at -2.54 2.54) (size 2.74 2.74) (drill 1.7) (layers "*.Cu" "*.Mask") (remove_unused_layers no) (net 2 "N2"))
  (pad "2" thru_hole circle (at 2.54 -2.54) (size 2.74 2.74) (drill 1.7) (layers "*.Cu" "*.Mask") (remove_unused_layers no) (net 2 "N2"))
  (pad "2" thru_hole circle (at 2.54 2.54) (size 2.74 2.74) (drill 1.7) (layers "*.Cu" "*.Mask") (remove_unused_layers no) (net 2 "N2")))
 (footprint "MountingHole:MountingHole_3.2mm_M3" (layer "F.Cu") (at 184.15 46.99)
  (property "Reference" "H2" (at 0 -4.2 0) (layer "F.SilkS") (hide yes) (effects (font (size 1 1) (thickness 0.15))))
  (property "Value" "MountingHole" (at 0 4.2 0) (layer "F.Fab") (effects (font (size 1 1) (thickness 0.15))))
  (pad "" np_thru_hole circle (at 0 0) (size 3.2 3.2) (drill 3.2) (layers "*.Cu" "*.Mask")))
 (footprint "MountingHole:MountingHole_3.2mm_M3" (layer "F.Cu") (at 133.35 85.09)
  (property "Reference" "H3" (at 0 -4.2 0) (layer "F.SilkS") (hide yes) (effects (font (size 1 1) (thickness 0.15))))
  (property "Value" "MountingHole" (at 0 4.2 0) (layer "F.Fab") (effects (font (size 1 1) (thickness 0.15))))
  (pad "" np_thru_hole circle (at 0 0) (size 3.2 3.2) (drill 3.2) (layers "*.Cu" "*.Mask")))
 (gr_circle (center 163.638738 67.437) (end 170.638738 67.437) (stroke (width 0.1) (type default)) (fill none) (layer "F.SilkS"))
 (gr_circle (center 163.638738 67.437) (end 178.091338 74.2188) (stroke (width 0.1) (type default)) (fill none) (layer "F.SilkS"))
 (gr_rect (start 129.54 43.18) (end 187.96 88.9) (stroke (width 0.05) (type default)) (fill none) (layer "Edge.Cuts"))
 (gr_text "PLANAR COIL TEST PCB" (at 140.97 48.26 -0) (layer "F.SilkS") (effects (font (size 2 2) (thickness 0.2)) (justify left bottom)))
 (segment (start 146.5834 66.9798) (end 146.243 66.6394) (width 0.127) (layer "F.Cu") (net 2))
 (segment (start 146.243 66.6394) (end 145.415 66.6394) (width 0.127) (layer "F.Cu") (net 2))
 (segment (start 144.9222 66.1466) (end 145.415 66.6394) (width 0.254) (layer "F.Cu") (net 2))
 (segment (start 147.2438 66.9798) (end 146.5834 66.9798) (width 0.127) (layer "F.Cu") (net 2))
 (segment (start 141.7574 66.1466) (end 144.9222 66.1466) (width 0.254) (layer "F.Cu") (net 2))
 (via (at 147.2438 66.9798) (size 0.6) (drill 0.3) (layers "F.Cu" "B.Cu") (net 2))
 (segment (start 138.0794 66.1466) (end 137.9474 66.0146) (width 0.254) (layer "B.Cu") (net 2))
 (segment (start 147.7772 66.9798) (end 147.2438 66.9798) (width 0.127) (layer "B.Cu") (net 2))
 (segment (start 141.7574 66.1466) (end 138.0794 66.1466) (width 0.254) (layer "B.Cu") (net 2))
 (segment (start 132.8674 66.0146) (end 132.8674 71.0946) (width 0.254) (layer "B.Cu") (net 2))
 (segment (start 137.9474 66.0146) (end 132.8674 66.0146) (width 0.254) (layer "B.Cu") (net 2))
 (segment (start 132.8674 71.0946) (end 137.9474 71.0946) (width 0.254) (layer "B.Cu") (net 2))
 (segment (start 141.7574 68.6866) (end 145.2678 68.6866) (width 0.254) (layer "F.Cu") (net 1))
 (segment (start 145.2678 68.6866) (end 145.415 68.5394) (width 0.254) (layer "F.Cu") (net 1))
 (segment (start 141.7574 68.6866) (end 135.5394 68.6866) (width 0.254) (layer "F.Cu") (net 1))
 (segment (start 145.415 68.5394) (end 146.4716 68.5394) (width 0.127) (layer "F.Cu") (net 1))
 (segment (start 147.0312 67.9798) (end 147.7772 67.9798) (width 0.127) (layer "F.Cu") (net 1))
 (segment (start 146.4716 68.5394) (end 147.0312 67.9798) (width 0.127) (layer "F.Cu") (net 1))
 (segment (start 135.5394 68.6866) (end 135.4074 68.5546) (width 0.254) (layer "F.Cu") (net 1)))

